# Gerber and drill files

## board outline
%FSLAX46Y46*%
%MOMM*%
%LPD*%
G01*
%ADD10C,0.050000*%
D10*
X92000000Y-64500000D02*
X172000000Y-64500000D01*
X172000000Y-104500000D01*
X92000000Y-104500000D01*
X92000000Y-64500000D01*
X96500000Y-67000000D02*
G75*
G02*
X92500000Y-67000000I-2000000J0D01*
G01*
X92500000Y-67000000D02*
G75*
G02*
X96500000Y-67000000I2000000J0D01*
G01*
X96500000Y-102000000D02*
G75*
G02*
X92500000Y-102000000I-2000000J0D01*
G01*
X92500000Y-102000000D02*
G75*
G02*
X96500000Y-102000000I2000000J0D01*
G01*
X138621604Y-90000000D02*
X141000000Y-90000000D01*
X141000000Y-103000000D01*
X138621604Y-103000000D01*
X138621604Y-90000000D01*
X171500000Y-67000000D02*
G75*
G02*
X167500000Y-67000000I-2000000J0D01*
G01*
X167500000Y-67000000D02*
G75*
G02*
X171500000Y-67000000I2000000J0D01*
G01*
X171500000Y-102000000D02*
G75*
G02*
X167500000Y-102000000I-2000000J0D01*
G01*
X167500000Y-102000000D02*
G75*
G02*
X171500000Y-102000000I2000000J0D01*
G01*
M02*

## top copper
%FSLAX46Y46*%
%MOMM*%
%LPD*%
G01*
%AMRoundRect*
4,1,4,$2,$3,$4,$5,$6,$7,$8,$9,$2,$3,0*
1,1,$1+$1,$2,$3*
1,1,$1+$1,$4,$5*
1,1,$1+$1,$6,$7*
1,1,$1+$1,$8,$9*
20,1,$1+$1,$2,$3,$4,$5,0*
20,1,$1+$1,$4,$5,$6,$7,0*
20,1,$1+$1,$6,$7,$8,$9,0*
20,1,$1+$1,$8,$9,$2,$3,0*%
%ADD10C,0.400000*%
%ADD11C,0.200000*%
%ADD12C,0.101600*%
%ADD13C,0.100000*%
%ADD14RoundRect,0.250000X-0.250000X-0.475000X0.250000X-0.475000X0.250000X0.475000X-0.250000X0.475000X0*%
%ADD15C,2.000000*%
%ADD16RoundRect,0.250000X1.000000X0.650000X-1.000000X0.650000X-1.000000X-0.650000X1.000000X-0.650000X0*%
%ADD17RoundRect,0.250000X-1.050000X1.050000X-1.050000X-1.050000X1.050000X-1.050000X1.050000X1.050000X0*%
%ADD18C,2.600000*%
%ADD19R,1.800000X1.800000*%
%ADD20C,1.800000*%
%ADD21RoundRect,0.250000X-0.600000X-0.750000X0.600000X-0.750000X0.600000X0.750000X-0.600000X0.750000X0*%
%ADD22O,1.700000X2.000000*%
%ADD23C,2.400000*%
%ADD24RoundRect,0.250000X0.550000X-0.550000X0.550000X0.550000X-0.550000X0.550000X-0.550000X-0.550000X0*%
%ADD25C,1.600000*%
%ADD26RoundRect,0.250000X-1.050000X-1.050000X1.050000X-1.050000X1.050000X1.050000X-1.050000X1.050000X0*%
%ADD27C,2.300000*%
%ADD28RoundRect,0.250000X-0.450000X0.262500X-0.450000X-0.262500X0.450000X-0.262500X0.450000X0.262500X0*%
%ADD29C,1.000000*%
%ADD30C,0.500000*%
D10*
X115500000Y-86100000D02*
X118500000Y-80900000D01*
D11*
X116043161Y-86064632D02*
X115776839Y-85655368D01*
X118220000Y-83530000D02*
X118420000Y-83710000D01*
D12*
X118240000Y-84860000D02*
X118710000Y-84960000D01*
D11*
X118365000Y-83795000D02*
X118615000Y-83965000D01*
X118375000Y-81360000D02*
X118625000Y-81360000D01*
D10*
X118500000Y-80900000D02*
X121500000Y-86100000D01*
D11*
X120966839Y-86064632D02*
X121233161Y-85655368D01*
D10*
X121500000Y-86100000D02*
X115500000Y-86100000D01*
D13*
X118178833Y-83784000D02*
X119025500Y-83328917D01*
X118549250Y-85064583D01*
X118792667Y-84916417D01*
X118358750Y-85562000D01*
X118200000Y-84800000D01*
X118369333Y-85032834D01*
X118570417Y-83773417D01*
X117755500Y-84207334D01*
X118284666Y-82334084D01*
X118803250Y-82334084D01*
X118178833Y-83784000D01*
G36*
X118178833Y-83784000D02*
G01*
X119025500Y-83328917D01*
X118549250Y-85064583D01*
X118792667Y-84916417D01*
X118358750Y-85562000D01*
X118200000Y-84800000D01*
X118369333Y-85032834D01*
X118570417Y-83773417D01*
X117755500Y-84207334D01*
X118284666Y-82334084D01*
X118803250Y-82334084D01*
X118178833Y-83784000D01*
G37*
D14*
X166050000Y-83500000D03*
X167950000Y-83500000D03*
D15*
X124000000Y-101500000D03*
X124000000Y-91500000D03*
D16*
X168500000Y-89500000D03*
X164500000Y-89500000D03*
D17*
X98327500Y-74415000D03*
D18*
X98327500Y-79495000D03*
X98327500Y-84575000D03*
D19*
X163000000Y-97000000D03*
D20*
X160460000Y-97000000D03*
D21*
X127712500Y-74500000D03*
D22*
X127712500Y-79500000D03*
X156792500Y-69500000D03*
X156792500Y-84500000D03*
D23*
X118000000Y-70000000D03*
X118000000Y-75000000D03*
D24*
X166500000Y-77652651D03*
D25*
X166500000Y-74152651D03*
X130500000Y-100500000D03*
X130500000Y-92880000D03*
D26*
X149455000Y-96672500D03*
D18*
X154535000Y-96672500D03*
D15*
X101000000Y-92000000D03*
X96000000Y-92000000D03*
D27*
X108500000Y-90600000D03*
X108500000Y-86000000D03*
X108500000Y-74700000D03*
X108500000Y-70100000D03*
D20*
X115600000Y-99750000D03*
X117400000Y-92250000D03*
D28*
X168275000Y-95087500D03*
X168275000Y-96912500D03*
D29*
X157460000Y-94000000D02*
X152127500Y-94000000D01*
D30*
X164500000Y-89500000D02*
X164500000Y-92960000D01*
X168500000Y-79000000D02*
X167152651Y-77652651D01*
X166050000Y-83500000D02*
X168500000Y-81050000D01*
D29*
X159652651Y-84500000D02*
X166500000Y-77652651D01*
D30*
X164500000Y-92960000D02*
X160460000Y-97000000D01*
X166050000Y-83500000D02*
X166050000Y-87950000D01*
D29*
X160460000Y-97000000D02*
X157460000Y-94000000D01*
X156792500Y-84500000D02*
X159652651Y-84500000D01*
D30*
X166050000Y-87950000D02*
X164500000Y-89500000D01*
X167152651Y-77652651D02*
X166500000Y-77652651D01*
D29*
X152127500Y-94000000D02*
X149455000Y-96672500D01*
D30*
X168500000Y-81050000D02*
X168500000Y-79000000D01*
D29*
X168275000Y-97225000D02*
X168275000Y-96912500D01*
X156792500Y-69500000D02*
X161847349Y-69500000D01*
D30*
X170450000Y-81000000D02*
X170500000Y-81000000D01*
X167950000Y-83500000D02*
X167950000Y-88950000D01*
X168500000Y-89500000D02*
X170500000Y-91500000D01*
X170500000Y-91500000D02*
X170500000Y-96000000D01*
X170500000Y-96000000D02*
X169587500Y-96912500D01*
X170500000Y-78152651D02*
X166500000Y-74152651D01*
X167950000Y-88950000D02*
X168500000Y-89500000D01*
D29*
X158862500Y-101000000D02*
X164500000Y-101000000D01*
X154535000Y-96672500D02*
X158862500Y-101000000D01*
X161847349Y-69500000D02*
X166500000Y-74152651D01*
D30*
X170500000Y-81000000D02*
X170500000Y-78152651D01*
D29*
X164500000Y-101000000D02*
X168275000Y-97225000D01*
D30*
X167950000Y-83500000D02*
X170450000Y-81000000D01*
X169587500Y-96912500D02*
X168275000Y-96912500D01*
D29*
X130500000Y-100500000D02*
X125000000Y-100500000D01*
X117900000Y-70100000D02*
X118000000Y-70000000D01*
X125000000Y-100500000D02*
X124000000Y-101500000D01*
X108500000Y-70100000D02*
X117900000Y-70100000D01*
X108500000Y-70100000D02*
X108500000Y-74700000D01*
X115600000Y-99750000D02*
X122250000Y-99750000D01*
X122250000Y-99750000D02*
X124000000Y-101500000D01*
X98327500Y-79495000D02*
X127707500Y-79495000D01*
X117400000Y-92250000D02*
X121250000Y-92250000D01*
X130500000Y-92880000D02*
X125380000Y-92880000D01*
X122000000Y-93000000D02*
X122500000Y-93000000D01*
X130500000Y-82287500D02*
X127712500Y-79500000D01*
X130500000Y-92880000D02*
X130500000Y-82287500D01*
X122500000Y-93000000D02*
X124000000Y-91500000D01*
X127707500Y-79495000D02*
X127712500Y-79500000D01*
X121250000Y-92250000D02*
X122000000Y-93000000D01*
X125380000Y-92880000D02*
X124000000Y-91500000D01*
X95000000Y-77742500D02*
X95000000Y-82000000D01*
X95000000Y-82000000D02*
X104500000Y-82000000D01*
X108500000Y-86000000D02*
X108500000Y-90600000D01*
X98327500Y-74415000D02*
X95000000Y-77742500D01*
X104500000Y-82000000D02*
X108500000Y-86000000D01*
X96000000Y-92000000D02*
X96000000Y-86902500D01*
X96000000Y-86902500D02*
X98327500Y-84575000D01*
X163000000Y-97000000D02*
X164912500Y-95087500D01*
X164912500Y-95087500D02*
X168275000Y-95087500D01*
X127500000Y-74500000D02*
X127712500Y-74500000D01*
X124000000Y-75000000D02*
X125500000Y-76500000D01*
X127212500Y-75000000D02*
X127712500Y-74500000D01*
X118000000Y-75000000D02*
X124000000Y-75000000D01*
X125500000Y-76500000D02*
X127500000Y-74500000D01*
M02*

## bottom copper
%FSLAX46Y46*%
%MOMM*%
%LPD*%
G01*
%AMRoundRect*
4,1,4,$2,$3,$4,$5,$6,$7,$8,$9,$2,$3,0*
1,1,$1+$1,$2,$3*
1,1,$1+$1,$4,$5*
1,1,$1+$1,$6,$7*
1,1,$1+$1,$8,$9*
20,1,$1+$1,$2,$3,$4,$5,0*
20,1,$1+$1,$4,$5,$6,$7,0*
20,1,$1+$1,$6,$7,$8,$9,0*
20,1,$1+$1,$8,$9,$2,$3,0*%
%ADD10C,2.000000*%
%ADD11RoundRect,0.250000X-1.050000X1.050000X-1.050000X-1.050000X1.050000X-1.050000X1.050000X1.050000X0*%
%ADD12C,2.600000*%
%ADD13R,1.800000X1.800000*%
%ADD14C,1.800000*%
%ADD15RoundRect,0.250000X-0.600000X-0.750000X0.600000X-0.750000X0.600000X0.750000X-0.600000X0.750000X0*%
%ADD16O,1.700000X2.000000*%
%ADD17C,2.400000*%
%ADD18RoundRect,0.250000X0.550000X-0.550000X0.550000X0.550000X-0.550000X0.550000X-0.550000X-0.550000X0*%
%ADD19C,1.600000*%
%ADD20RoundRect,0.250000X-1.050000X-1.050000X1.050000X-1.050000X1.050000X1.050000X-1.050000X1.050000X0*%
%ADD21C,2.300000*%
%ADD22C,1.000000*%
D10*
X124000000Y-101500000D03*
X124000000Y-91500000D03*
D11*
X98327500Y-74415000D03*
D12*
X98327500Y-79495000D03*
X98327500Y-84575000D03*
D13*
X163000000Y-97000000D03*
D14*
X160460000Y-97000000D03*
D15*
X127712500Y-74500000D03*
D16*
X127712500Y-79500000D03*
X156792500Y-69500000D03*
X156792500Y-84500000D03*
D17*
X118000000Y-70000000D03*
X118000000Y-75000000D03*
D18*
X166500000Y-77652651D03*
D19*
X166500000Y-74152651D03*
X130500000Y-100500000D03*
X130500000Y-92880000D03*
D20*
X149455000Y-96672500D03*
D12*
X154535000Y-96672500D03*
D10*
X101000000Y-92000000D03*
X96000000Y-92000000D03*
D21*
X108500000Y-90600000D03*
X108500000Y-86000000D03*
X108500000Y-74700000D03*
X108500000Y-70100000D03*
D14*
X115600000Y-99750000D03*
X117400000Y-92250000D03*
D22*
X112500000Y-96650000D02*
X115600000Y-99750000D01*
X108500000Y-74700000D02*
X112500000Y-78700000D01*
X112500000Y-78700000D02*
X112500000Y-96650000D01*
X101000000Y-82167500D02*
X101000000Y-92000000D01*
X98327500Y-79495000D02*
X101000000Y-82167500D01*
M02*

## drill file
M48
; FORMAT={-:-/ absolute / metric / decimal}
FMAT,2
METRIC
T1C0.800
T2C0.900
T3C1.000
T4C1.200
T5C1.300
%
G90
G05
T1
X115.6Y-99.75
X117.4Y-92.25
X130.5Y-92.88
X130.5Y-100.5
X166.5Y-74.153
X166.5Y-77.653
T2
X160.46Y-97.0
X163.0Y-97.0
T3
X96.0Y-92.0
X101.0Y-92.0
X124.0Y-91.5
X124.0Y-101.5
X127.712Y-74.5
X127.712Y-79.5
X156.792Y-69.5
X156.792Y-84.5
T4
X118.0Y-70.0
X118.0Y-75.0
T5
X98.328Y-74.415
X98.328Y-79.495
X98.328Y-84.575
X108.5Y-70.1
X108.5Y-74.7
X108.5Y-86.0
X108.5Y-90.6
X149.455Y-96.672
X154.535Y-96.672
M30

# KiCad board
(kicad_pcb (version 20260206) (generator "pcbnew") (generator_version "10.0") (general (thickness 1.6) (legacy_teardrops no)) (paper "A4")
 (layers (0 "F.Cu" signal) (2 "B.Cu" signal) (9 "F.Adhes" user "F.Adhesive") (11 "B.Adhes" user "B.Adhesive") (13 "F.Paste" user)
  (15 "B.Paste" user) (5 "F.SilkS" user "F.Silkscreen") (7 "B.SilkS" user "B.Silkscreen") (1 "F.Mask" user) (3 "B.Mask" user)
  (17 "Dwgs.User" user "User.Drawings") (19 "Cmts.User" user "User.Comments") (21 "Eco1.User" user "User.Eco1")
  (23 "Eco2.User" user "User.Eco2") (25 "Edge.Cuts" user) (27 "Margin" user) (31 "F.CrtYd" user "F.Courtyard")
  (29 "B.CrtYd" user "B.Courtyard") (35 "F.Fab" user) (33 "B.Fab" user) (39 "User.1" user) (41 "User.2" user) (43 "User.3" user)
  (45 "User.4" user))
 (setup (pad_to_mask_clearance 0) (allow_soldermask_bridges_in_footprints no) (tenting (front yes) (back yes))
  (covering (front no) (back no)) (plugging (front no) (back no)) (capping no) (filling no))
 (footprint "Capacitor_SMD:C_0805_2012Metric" (layer "F.Cu") (at 167 83.5)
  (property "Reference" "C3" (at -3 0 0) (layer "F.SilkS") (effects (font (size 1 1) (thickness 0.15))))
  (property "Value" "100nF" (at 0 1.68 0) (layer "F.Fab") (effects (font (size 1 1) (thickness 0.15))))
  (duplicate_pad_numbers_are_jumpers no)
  (pad "1" smd roundrect (at -0.95 0) (size 1 1.45) (layers "F.Cu" "F.Mask" "F.Paste") (roundrect_rratio 0.25) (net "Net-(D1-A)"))
  (pad "2" smd roundrect (at 0.95 0) (size 1 1.45) (layers "F.Cu" "F.Mask" "F.Paste") (roundrect_rratio 0.25) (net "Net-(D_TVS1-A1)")))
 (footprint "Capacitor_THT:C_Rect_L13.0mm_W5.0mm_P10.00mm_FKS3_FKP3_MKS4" (layer "F.Cu") (at 124 101.5 90)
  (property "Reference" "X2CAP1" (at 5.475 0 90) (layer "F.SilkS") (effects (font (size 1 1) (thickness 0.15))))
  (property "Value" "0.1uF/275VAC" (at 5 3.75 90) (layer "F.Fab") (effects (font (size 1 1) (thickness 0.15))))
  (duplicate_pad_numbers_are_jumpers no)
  (pad "1" thru_hole circle (at 0 0 90) (size 2 2) (drill 1) (layers "*.Cu" "*.Mask") (remove_unused_layers no) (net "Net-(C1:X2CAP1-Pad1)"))
  (pad "2" thru_hole circle (at 10 0 90) (size 2 2) (drill 1) (layers "*.Cu" "*.Mask") (remove_unused_layers no) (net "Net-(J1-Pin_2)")))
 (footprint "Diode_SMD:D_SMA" (layer "F.Cu") (at 166.5 89.5 180)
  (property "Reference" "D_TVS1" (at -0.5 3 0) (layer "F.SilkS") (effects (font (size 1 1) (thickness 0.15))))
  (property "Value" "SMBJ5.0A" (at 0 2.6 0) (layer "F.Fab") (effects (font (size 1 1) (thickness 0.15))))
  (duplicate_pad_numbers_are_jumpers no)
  (pad "1" smd roundrect (at -2 0 180) (size 2.5 1.8) (layers "F.Cu" "F.Mask" "F.Paste") (roundrect_rratio 0.1388888889)
   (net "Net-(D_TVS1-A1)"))
  (pad "2" smd roundrect (at 2 0 180) (size 2.5 1.8) (layers "F.Cu" "F.Mask" "F.Paste") (roundrect_rratio 0.1388888889) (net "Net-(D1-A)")))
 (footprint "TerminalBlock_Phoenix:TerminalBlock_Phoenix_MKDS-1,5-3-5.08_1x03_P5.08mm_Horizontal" (layer "F.Cu") (at 98.3275 74.415 -90)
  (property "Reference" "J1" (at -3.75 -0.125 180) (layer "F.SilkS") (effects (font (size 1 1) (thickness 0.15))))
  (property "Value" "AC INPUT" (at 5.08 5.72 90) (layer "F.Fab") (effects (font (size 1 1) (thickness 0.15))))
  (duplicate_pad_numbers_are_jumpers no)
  (pad "1" thru_hole roundrect (at 0 0 270) (size 2.6 2.6) (drill 1.3) (layers "*.Cu" "*.Mask") (remove_unused_layers no)
   (roundrect_rratio 0.096154) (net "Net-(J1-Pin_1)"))
  (pad "2" thru_hole circle (at 5.08 0 270) (size 2.6 2.6) (drill 1.3) (layers "*.Cu" "*.Mask") (remove_unused_layers no)
   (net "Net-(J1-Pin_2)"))
  (pad "3" thru_hole circle (at 10.16 0 270) (size 2.6 2.6) (drill 1.3) (layers "*.Cu" "*.Mask") (remove_unused_layers no) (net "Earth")))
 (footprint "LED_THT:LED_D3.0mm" (layer "F.Cu") (at 163 97 180)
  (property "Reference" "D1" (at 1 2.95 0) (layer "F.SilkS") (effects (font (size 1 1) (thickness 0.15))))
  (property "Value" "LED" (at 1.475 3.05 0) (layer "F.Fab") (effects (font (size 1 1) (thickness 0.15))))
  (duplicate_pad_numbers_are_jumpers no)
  (pad "1" thru_hole rect (at 0 0 180) (size 1.8 1.8) (drill 0.9) (layers "*.Cu" "*.Mask") (remove_unused_layers no) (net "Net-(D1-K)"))
  (pad "2" thru_hole circle (at 2.54 0 180) (size 1.8 1.8) (drill 0.9) (layers "*.Cu" "*.Mask") (remove_unused_layers no) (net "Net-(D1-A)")))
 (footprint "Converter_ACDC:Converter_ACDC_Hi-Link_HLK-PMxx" (layer "F.Cu") (at 127.7125 74.5)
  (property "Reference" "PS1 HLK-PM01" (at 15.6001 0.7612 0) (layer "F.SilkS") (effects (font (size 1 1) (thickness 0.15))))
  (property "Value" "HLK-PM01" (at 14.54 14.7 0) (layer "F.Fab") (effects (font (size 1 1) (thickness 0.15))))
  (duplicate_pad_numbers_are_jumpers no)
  (pad "1" thru_hole roundrect (at 0 0) (size 1.7 2) (drill 1) (layers "*.Cu" "*.Mask") (remove_unused_layers no)
   (roundrect_rratio 0.147059) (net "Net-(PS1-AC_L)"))
  (pad "2" thru_hole oval (at 0 5) (size 1.7 2) (drill 1) (layers "*.Cu" "*.Mask") (remove_unused_layers no) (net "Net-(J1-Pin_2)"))
  (pad "3" thru_hole oval (at 29.08 -5) (size 1.7 2) (drill 1) (layers "*.Cu" "*.Mask") (remove_unused_layers no) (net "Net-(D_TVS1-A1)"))
  (pad "4" thru_hole oval (at 29.08 10) (size 1.7 2) (drill 1) (layers "*.Cu" "*.Mask") (remove_unused_layers no) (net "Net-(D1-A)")))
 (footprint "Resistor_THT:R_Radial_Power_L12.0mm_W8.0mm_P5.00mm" (layer "F.Cu") (at 118 70 -90)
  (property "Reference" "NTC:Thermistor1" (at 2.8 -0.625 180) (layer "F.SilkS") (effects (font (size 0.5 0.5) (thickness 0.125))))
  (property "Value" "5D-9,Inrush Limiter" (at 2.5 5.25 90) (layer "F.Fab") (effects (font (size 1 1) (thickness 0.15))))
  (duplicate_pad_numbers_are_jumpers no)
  (pad "1" thru_hole circle (at 0 0 270) (size 2.4 2.4) (drill 1.2) (layers "*.Cu" "*.Mask") (remove_unused_layers no)
   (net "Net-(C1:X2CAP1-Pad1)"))
  (pad "2" thru_hole circle (at 5 0 270) (size 2.4 2.4) (drill 1.2) (layers "*.Cu" "*.Mask") (remove_unused_layers no)
   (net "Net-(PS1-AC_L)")))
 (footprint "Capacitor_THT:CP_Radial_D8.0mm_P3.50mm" (layer "F.Cu") (at 166.5 77.652651 90)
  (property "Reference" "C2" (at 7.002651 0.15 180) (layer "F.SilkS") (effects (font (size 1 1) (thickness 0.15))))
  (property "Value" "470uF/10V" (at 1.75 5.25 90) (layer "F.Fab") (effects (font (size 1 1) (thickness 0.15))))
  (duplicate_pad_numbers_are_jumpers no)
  (pad "1" thru_hole roundrect (at 0 0 90) (size 1.6 1.6) (drill 0.8) (layers "*.Cu" "*.Mask") (remove_unused_layers no)
   (roundrect_rratio 0.15625) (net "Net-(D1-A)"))
  (pad "2" thru_hole circle (at 3.5 0 90) (size 1.6 1.6) (drill 0.8) (layers "*.Cu" "*.Mask") (remove_unused_layers no)
   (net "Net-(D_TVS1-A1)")))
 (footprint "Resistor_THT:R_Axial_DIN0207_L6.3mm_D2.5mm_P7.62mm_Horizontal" (layer "F.Cu") (at 130.5 100.5 90)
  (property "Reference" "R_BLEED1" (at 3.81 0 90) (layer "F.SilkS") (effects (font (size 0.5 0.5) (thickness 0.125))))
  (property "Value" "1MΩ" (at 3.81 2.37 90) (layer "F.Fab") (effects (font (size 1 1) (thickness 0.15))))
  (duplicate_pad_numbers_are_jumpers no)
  (pad "1" thru_hole circle (at 0 0 90) (size 1.6 1.6) (drill 0.8) (layers "*.Cu" "*.Mask") (remove_unused_layers no)
   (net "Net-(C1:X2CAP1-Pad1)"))
  (pad "2" thru_hole circle (at 7.62 0 90) (size 1.6 1.6) (drill 0.8) (layers "*.Cu" "*.Mask") (remove_unused_layers no)
   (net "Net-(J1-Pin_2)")))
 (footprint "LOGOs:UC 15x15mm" (layer "F.Cu") (at 105 97.5)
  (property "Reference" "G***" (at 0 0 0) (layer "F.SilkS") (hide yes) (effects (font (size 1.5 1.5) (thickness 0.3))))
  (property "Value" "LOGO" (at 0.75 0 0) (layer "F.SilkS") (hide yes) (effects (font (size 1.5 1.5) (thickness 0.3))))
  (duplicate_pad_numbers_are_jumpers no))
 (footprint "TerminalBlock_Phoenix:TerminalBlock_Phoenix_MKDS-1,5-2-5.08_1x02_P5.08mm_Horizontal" (layer "F.Cu") (at 149.455 96.6725)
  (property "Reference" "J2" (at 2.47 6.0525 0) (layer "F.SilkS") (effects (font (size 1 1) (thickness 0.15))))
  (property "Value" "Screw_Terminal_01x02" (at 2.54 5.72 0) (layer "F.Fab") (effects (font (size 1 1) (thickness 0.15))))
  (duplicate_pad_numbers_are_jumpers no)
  (pad "1" thru_hole roundrect (at 0 0) (size 2.6 2.6) (drill 1.3) (layers "*.Cu" "*.Mask") (remove_unused_layers no)
   (roundrect_rratio 0.096154) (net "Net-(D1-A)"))
  (pad "2" thru_hole circle (at 5.08 0) (size 2.6 2.6) (drill 1.3) (layers "*.Cu" "*.Mask") (remove_unused_layers no)
   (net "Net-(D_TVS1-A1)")))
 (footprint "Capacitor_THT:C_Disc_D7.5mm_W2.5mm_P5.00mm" (layer "F.Cu") (at 101 92 180)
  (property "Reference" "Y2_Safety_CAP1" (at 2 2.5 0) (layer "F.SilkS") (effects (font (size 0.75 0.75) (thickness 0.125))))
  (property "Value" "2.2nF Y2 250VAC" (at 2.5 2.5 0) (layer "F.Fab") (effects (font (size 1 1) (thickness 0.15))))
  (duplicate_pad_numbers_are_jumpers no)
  (pad "1" thru_hole circle (at 0 0 180) (size 2 2) (drill 1) (layers "*.Cu" "*.Mask") (remove_unused_layers no) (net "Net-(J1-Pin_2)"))
  (pad "2" thru_hole circle (at 5 0 180) (size 2 2) (drill 1) (layers "*.Cu" "*.Mask") (remove_unused_layers no) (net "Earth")))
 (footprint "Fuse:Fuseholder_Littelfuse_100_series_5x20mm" (layer "F.Cu") (at 108.5 90.6 90)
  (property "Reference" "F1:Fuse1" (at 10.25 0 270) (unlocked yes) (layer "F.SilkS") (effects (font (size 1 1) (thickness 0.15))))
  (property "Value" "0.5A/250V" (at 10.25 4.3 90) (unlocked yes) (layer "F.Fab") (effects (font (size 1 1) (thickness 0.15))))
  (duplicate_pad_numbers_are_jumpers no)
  (pad "1" thru_hole circle (at 0 0 90) (size 2.3 2.3) (drill 1.3) (layers "*.Cu" "*.Mask") (remove_unused_layers no) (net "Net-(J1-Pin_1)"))
  (pad "1" thru_hole circle (at 4.6 0 90) (size 2.3 2.3) (drill 1.3) (layers "*.Cu" "*.Mask") (remove_unused_layers no)
   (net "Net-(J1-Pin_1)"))
  (pad "2" thru_hole circle (at 15.9 0 90) (size 2.3 2.3) (drill 1.3) (layers "*.Cu" "*.Mask") (remove_unused_layers no)
   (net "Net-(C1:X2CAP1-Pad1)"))
  (pad "2" thru_hole circle (at 20.5 0 90) (size 2.3 2.3) (drill 1.3) (layers "*.Cu" "*.Mask") (remove_unused_layers no)
   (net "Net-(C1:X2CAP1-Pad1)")))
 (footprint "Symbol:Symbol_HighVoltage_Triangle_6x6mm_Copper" (layer "F.Cu") (at 118.5 83.5)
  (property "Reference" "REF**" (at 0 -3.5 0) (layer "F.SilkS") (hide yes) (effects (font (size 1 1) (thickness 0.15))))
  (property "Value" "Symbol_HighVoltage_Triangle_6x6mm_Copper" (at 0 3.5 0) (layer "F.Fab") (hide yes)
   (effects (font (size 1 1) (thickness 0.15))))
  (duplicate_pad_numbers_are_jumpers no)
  (fp_line (start -3 2.6) (end 0 -2.6) (stroke (width 0.4) (type solid)) (layer "F.Cu"))
  (fp_line (start -2.456839 2.564632) (end -2.723161 2.155368) (stroke (width 0.2) (type default)) (layer "F.Cu"))
  (fp_line (start -0.28 0.03) (end -0.08 0.21) (stroke (width 0.2) (type default)) (layer "F.Cu"))
  (fp_line (start -0.26 1.36) (end 0.21 1.46) (stroke (width 0.1016) (type default)) (layer "F.Cu"))
  (fp_line (start -0.135 0.295) (end 0.115 0.465) (stroke (width 0.2) (type default)) (layer "F.Cu"))
  (fp_line (start -0.125 -2.14) (end 0.125 -2.14) (stroke (width 0.2) (type default)) (layer "F.Cu"))
  (fp_line (start 0 -2.6) (end 3 2.6) (stroke (width 0.4) (type solid)) (layer "F.Cu"))
  (fp_line (start 2.466839 2.564632) (end 2.733161 2.155368) (stroke (width 0.2) (type default)) (layer "F.Cu"))
  (fp_line (start 3 2.6) (end -3 2.6) (stroke (width 0.4) (type solid)) (layer "F.Cu"))
  (fp_poly
   (pts (xy -0.321167 0.284) (xy 0.5255 -0.171083) (xy 0.04925 1.564583) (xy 0.292667 1.416417) (xy -0.14125 2.062) (xy -0.3 1.3)
    (xy -0.130667 1.532834) (xy 0.070417 0.273417) (xy -0.7445 0.707334) (xy -0.215334 -1.165916) (xy 0.30325 -1.165916))
   (stroke (width 0.1) (type solid)) (fill yes) (layer "F.Cu")))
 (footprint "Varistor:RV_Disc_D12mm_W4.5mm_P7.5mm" (layer "F.Cu") (at 115.6 99.75 90)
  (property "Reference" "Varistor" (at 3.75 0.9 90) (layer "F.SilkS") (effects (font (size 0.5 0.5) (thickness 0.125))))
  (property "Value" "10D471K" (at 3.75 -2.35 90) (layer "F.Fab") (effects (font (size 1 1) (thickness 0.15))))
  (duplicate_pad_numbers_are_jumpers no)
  (pad "1" thru_hole circle (at 0 0 90) (size 1.8 1.8) (drill 0.8) (layers "*.Cu" "*.Mask") (remove_unused_layers no)
   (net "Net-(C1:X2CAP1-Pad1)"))
  (pad "2" thru_hole circle (at 7.5 1.8 90) (size 1.8 1.8) (drill 0.8) (layers "*.Cu" "*.Mask") (remove_unused_layers no)
   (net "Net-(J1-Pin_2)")))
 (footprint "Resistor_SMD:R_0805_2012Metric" (layer "F.Cu") (at 168.275 96 -90)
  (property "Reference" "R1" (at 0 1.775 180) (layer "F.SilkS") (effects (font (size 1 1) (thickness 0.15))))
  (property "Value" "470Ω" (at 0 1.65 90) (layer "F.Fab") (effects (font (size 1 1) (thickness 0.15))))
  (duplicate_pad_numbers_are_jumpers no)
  (pad "1" smd roundrect (at -0.9125 0 270) (size 1.025 1.4) (layers "F.Cu" "F.Mask" "F.Paste") (roundrect_rratio 0.243902)
   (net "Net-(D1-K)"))
  (pad "2" smd roundrect (at 0.9125 0 270) (size 1.025 1.4) (layers "F.Cu" "F.Mask" "F.Paste") (roundrect_rratio 0.243902)
   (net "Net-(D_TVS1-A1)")))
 (gr_rect (start 92 64.5) (end 172 104.5) (stroke (width 0.05) (type default)) (fill no) (layer "Edge.Cuts"))
 (gr_circle (center 94.5 67) (end 96.5 67) (stroke (width 0.05) (type default)) (fill no) (layer "Edge.Cuts"))
 (gr_circle (center 94.5 102) (end 96.5 102) (stroke (width 0.05) (type default)) (fill no) (layer "Edge.Cuts"))
 (gr_rect (start 138.621604 90) (end 141 103) (stroke (width 0.05) (type default)) (fill no) (layer "Edge.Cuts"))
 (gr_circle (center 169.5 67) (end 171.5 67) (stroke (width 0.05) (type default)) (fill no) (layer "Edge.Cuts"))
 (gr_circle (center 169.5 102) (end 171.5 102) (stroke (width 0.05) (type default)) (fill no) (layer "Edge.Cuts"))
 (segment (start 157.46 94) (end 152.1275 94) (width 1) (layer "F.Cu") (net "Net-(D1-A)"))
 (segment (start 164.5 89.5) (end 164.5 92.96) (width 0.5) (layer "F.Cu") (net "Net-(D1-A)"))
 (segment (start 168.5 79) (end 167.152651 77.652651) (width 0.5) (layer "F.Cu") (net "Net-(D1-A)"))
 (segment (start 166.05 83.5) (end 168.5 81.05) (width 0.5) (layer "F.Cu") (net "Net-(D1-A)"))
 (segment (start 159.652651 84.5) (end 166.5 77.652651) (width 1) (layer "F.Cu") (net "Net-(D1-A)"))
 (segment (start 164.5 92.96) (end 160.46 97) (width 0.5) (layer "F.Cu") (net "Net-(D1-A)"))
 (segment (start 166.05 83.5) (end 166.05 87.95) (width 0.5) (layer "F.Cu") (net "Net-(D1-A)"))
 (segment (start 160.46 97) (end 157.46 94) (width 1) (layer "F.Cu") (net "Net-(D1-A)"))
 (segment (start 156.7925 84.5) (end 159.652651 84.5) (width 1) (layer "F.Cu") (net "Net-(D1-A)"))
 (segment (start 166.05 87.95) (end 164.5 89.5) (width 0.5) (layer "F.Cu") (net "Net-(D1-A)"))
 (segment (start 167.152651 77.652651) (end 166.5 77.652651) (width 0.5) (layer "F.Cu") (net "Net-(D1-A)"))
 (segment (start 152.1275 94) (end 149.455 96.6725) (width 1) (layer "F.Cu") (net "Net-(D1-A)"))
 (segment (start 168.5 81.05) (end 168.5 79) (width 0.5) (layer "F.Cu") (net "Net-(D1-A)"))
 (segment (start 168.275 97.225) (end 168.275 96.9125) (width 1) (layer "F.Cu") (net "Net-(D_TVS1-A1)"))
 (segment (start 156.7925 69.5) (end 161.847349 69.5) (width 1) (layer "F.Cu") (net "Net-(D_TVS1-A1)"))
 (segment (start 170.45 81) (end 170.5 81) (width 0.5) (layer "F.Cu") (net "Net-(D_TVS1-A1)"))
 (segment (start 167.95 83.5) (end 167.95 88.95) (width 0.5) (layer "F.Cu") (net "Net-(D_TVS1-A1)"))
 (segment (start 168.5 89.5) (end 170.5 91.5) (width 0.5) (layer "F.Cu") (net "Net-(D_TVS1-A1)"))
 (segment (start 170.5 91.5) (end 170.5 96) (width 0.5) (layer "F.Cu") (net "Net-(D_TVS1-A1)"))
 (segment (start 170.5 96) (end 169.5875 96.9125) (width 0.5) (layer "F.Cu") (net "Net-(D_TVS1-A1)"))
 (segment (start 170.5 78.152651) (end 166.5 74.152651) (width 0.5) (layer "F.Cu") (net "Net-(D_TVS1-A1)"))
 (segment (start 167.95 88.95) (end 168.5 89.5) (width 0.5) (layer "F.Cu") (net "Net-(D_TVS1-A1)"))
 (segment (start 158.8625 101) (end 164.5 101) (width 1) (layer "F.Cu") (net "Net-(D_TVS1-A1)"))
 (segment (start 154.535 96.6725) (end 158.8625 101) (width 1) (layer "F.Cu") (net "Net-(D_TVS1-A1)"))
 (segment (start 161.847349 69.5) (end 166.5 74.152651) (width 1) (layer "F.Cu") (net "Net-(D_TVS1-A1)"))
 (segment (start 170.5 81) (end 170.5 78.152651) (width 0.5) (layer "F.Cu") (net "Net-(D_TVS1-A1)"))
 (segment (start 164.5 101) (end 168.275 97.225) (width 1) (layer "F.Cu") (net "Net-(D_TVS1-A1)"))
 (segment (start 167.95 83.5) (end 170.45 81) (width 0.5) (layer "F.Cu") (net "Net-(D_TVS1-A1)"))
 (segment (start 169.5875 96.9125) (end 168.275 96.9125) (width 0.5) (layer "F.Cu") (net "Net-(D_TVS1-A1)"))
 (segment (start 130.5 100.5) (end 125 100.5) (width 1) (layer "F.Cu") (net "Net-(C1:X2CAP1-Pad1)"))
 (segment (start 117.9 70.1) (end 118 70) (width 1) (layer "F.Cu") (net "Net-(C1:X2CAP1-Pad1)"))
 (segment (start 125 100.5) (end 124 101.5) (width 1) (layer "F.Cu") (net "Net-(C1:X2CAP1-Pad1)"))
 (segment (start 108.5 70.1) (end 117.9 70.1) (width 1) (layer "F.Cu") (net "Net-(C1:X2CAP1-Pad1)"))
 (segment (start 108.5 70.1) (end 108.5 74.7) (width 1) (layer "F.Cu") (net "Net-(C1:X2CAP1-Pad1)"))
 (segment (start 115.6 99.75) (end 122.25 99.75) (width 1) (layer "F.Cu") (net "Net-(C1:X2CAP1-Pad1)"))
 (segment (start 122.25 99.75) (end 124 101.5) (width 1) (layer "F.Cu") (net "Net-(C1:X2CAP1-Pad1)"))
 (segment (start 112.5 96.65) (end 115.6 99.75) (width 1) (layer "B.Cu") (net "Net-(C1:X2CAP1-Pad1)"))
 (segment (start 108.5 74.7) (end 112.5 78.7) (width 1) (layer "B.Cu") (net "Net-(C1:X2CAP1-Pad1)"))
 (segment (start 112.5 78.7) (end 112.5 96.65) (width 1) (layer "B.Cu") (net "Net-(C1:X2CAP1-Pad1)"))
 (segment (start 98.3275 79.495) (end 127.7075 79.495) (width 1) (layer "F.Cu") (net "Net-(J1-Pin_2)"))
 (segment (start 117.4 92.25) (end 121.25 92.25) (width 1) (layer "F.Cu") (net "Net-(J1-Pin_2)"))
 (segment (start 130.5 92.88) (end 125.38 92.88) (width 1) (layer "F.Cu") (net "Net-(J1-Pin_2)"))
 (segment (start 122 93) (end 122.5 93) (width 1) (layer "F.Cu") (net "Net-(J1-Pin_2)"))
 (segment (start 130.5 82.2875) (end 127.7125 79.5) (width 1) (layer "F.Cu") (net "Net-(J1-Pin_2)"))
 (segment (start 130.5 92.88) (end 130.5 82.2875) (width 1) (layer "F.Cu") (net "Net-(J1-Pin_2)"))
 (segment (start 122.5 93) (end 124 91.5) (width 1) (layer "F.Cu") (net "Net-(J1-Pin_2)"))
 (segment (start 127.7075 79.495) (end 127.7125 79.5) (width 1) (layer "F.Cu") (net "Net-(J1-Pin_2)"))
 (segment (start 121.25 92.25) (end 122 93) (width 1) (layer "F.Cu") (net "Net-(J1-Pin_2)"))
 (segment (start 125.38 92.88) (end 124 91.5) (width 1) (layer "F.Cu") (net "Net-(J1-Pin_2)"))
 (segment (start 101 82.1675) (end 101 92) (width 1) (layer "B.Cu") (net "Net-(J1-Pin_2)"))
 (segment (start 98.3275 79.495) (end 101 82.1675) (width 1) (layer "B.Cu") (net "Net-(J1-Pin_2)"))
 (segment (start 95 77.7425) (end 95 82) (width 1) (layer "F.Cu") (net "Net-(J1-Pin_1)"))
 (segment (start 95 82) (end 104.5 82) (width 1) (layer "F.Cu") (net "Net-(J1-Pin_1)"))
 (segment (start 108.5 86) (end 108.5 90.6) (width 1) (layer "F.Cu") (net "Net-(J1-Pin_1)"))
 (segment (start 98.3275 74.415) (end 95 77.7425) (width 1) (layer "F.Cu") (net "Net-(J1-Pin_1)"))
 (segment (start 104.5 82) (end 108.5 86) (width 1) (layer "F.Cu") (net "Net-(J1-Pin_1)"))
 (segment (start 96 92) (end 96 86.9025) (width 1) (layer "F.Cu") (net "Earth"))
 (segment (start 96 86.9025) (end 98.3275 84.575) (width 1) (layer "F.Cu") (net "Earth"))
 (segment (start 163 97) (end 164.9125 95.0875) (width 1) (layer "F.Cu") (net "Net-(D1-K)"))
 (segment (start 164.9125 95.0875) (end 168.275 95.0875) (width 1) (layer "F.Cu") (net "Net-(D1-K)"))
 (segment (start 127.5 74.5) (end 127.7125 74.5) (width 1) (layer "F.Cu") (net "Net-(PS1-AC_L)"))
 (segment (start 124 75) (end 125.5 76.5) (width 1) (layer "F.Cu") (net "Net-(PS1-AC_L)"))
 (segment (start 127.2125 75) (end 127.7125 74.5) (width 1) (layer "F.Cu") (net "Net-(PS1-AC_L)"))
 (segment (start 118 75) (end 124 75) (width 1) (layer "F.Cu") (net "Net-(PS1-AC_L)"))
 (segment (start 125.5 76.5) (end 127.5 74.5) (width 1) (layer "F.Cu") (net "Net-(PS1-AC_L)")))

